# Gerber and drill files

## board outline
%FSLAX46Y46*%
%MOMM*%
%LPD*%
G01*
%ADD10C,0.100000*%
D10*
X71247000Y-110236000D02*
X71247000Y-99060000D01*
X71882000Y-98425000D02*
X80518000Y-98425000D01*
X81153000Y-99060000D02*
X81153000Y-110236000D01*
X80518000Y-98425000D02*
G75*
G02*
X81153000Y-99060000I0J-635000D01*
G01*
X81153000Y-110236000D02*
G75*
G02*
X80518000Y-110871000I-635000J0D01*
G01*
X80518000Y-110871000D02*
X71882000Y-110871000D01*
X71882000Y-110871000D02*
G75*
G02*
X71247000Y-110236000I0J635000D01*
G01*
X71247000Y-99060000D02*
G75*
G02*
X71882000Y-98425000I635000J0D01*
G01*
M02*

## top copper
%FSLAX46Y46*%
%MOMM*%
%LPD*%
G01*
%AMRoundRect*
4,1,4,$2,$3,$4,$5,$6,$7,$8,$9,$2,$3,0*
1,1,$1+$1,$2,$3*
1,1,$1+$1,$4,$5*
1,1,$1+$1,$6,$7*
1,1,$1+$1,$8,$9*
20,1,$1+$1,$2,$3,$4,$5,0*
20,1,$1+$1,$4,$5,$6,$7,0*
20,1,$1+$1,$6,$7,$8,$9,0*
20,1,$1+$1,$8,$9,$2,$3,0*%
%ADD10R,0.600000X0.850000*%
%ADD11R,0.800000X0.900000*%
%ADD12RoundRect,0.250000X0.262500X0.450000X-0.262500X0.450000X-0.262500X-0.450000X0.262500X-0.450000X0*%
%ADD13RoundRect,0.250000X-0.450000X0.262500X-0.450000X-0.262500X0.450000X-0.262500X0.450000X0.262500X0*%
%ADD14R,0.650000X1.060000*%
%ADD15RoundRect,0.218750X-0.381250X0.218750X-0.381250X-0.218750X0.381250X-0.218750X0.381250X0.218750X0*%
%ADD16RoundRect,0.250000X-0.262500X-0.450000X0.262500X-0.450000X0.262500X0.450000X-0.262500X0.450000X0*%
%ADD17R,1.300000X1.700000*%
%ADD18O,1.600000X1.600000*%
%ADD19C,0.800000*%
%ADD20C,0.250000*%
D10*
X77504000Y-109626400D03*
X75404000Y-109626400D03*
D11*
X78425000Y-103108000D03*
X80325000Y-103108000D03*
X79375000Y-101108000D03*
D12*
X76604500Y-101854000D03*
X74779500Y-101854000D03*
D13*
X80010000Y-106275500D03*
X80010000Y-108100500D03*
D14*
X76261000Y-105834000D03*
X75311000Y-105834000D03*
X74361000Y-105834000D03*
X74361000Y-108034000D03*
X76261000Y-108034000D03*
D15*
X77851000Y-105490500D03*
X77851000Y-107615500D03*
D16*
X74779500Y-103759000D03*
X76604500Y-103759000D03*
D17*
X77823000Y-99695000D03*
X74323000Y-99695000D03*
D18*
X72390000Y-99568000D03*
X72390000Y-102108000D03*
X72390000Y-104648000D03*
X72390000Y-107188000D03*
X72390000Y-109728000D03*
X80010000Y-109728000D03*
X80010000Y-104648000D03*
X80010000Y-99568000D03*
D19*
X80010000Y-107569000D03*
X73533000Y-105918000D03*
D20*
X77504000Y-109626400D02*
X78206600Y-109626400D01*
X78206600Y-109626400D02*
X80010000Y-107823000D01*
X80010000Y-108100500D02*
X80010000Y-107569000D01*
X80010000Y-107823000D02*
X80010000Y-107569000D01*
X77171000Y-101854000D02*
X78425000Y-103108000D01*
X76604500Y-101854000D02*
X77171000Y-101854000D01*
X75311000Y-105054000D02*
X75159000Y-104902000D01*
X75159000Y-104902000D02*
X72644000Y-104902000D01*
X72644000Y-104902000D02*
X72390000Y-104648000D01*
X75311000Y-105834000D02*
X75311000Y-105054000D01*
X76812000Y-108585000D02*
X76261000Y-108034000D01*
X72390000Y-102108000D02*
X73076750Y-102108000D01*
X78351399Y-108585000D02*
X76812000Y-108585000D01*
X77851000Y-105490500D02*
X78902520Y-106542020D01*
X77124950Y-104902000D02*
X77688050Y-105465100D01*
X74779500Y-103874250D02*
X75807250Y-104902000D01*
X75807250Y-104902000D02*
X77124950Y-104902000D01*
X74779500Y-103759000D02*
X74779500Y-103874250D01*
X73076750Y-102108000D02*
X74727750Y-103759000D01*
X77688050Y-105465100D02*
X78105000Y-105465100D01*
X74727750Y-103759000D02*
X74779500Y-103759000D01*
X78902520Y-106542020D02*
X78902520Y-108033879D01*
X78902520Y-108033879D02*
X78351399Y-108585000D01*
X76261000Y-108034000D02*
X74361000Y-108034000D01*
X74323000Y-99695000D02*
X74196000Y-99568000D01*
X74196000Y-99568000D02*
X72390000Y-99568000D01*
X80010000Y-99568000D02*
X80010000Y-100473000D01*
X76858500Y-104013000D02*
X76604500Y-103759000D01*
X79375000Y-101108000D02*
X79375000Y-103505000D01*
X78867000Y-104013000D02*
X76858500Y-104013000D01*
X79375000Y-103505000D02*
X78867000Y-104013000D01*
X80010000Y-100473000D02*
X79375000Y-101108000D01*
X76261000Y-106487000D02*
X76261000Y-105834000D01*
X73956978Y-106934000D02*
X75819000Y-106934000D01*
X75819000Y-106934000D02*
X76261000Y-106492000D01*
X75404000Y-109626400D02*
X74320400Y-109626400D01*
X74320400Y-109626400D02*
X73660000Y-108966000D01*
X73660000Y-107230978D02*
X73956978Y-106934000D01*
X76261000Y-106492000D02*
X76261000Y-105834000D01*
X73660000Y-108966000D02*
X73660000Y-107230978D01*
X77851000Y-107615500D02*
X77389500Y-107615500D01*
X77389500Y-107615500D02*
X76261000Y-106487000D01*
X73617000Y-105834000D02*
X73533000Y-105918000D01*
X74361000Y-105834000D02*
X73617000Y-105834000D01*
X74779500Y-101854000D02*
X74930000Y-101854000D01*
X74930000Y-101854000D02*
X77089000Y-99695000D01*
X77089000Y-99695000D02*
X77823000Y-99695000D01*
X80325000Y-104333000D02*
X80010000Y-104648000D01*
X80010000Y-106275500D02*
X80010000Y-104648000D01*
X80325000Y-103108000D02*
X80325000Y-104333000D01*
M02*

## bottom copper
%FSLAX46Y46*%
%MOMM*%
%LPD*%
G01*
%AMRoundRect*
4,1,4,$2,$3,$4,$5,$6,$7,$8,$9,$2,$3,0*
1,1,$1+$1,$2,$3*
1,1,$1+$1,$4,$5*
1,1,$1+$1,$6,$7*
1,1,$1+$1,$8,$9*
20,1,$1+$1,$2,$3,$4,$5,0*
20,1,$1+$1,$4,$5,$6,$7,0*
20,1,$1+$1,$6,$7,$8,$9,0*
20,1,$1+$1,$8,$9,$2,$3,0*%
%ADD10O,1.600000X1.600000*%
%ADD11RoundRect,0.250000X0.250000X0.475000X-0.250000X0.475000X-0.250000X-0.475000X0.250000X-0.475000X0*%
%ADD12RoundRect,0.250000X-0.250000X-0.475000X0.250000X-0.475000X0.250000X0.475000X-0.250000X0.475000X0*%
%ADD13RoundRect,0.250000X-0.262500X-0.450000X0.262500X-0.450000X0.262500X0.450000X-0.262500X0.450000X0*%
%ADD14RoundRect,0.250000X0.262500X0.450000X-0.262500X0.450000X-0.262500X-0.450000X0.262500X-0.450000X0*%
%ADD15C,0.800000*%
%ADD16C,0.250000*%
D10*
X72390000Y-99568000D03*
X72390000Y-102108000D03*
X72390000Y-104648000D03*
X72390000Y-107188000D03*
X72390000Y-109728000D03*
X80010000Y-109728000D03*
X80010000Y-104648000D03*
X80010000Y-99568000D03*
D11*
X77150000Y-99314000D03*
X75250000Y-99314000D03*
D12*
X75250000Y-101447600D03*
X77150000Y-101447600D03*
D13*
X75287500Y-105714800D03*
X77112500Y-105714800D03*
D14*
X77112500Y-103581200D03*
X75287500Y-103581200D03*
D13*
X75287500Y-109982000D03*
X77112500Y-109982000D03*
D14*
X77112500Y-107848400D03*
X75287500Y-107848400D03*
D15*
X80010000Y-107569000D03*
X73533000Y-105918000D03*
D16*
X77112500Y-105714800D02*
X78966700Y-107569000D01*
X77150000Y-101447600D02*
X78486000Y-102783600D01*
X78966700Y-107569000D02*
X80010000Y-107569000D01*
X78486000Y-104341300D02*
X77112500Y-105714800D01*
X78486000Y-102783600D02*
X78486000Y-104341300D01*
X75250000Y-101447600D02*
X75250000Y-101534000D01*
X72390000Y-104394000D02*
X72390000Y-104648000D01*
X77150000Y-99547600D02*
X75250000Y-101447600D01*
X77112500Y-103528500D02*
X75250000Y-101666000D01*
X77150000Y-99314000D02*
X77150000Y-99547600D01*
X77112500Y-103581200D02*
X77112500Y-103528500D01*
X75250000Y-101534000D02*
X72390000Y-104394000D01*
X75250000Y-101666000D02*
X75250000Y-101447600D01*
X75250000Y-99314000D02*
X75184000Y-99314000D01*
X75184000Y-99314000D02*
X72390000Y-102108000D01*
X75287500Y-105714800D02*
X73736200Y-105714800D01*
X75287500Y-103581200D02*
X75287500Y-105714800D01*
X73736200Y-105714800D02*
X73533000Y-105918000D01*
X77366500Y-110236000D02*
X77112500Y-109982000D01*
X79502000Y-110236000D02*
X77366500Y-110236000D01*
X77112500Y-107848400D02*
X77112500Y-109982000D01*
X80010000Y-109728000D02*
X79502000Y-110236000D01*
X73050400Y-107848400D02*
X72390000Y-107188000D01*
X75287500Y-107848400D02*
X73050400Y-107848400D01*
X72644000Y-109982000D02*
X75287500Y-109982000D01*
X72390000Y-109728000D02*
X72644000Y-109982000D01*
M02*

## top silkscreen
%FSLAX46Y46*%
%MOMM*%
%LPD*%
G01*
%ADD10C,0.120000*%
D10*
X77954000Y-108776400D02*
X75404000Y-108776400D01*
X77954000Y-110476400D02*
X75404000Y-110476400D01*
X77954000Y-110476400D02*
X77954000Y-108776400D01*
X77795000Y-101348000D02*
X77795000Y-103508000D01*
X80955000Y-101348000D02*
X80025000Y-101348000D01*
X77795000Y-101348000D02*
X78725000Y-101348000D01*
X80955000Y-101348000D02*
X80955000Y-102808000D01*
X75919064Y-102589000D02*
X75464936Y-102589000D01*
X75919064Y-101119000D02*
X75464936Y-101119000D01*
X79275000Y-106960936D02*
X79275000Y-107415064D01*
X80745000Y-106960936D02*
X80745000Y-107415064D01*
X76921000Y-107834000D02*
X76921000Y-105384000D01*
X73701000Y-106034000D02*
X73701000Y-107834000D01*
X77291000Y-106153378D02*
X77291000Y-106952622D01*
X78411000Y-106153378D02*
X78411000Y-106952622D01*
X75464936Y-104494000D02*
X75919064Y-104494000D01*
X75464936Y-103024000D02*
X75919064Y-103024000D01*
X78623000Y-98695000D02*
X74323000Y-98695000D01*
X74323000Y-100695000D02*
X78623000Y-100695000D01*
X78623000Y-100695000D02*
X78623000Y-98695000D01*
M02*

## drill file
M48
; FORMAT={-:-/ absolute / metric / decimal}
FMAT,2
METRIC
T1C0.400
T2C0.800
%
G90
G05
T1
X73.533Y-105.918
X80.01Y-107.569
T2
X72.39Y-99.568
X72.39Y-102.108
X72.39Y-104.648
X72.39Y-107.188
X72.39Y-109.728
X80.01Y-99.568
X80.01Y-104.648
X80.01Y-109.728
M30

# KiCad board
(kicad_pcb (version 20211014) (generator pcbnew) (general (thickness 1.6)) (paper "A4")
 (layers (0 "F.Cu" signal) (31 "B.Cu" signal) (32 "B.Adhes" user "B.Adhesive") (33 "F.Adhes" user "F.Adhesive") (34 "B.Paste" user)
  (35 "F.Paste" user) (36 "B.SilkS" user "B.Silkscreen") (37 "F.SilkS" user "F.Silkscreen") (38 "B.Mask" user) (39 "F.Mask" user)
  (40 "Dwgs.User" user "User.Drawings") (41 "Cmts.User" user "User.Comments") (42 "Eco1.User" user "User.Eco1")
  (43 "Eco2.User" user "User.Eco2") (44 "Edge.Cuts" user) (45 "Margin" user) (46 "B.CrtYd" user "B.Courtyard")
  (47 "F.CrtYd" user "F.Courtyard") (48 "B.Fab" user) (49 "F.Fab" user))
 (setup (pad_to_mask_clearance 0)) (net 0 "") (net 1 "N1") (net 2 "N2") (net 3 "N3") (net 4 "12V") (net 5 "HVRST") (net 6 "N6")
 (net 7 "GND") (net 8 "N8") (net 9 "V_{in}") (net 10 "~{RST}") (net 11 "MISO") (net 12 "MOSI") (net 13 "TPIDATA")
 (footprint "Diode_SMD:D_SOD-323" (layer "F.Cu") (at 76.454 109.6264 180)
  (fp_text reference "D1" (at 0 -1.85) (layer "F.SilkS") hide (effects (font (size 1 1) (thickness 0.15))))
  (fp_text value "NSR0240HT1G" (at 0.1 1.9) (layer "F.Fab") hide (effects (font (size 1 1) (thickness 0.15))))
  (fp_line (start -1.5 0.85) (end 1.05 0.85) (layer "F.SilkS") (width 0.12))
  (fp_line (start -1.5 -0.85) (end 1.05 -0.85) (layer "F.SilkS") (width 0.12))
  (fp_line (start -1.5 -0.85) (end -1.5 0.85) (layer "F.SilkS") (width 0.12))
  (pad "1" smd rect locked (at -1.05 0 180) (size 0.6 0.85) (layers "F.Cu" "F.Paste" "F.Mask") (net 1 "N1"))
  (pad "2" smd rect locked (at 1.05 0 180) (size 0.6 0.85) (layers "F.Cu" "F.Paste" "F.Mask") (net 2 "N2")))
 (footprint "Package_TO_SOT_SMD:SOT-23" (layer "F.Cu") (at 79.375 102.108 90)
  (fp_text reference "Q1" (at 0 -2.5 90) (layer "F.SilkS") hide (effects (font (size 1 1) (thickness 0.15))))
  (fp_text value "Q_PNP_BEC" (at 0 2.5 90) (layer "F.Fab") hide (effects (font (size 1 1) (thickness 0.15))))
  (fp_line (start 0.76 -1.58) (end -1.4 -1.58) (layer "F.SilkS") (width 0.12))
  (fp_line (start 0.76 1.58) (end 0.76 0.65) (layer "F.SilkS") (width 0.12))
  (fp_line (start 0.76 -1.58) (end 0.76 -0.65) (layer "F.SilkS") (width 0.12))
  (fp_line (start 0.76 1.58) (end -0.7 1.58) (layer "F.SilkS") (width 0.12))
  (pad "1" smd rect locked (at -1 -0.95 90) (size 0.9 0.8) (layers "F.Cu" "F.Paste" "F.Mask") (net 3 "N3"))
  (pad "2" smd rect locked (at -1 0.95 90) (size 0.9 0.8) (layers "F.Cu" "F.Paste" "F.Mask") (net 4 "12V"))
  (pad "3" smd rect locked (at 1 0 90) (size 0.9 0.8) (layers "F.Cu" "F.Paste" "F.Mask") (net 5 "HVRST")))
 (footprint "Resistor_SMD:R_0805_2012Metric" (layer "F.Cu") (at 75.692 101.854 180)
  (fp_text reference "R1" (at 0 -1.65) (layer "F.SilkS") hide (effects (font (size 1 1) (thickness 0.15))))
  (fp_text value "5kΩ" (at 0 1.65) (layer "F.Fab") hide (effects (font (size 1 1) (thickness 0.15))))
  (fp_line (start -0.227064 -0.735) (end 0.227064 -0.735) (layer "F.SilkS") (width 0.12))
  (fp_line (start -0.227064 0.735) (end 0.227064 0.735) (layer "F.SilkS") (width 0.12))
  (pad "1" smd roundrect locked (at -0.9125 0 180) (size 1.025 1.4) (layers "F.Cu" "F.Paste" "F.Mask") (roundrect_rratio 0.243902)
   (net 3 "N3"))
  (pad "2" smd roundrect locked (at 0.9125 0 180) (size 1.025 1.4) (layers "F.Cu" "F.Paste" "F.Mask") (roundrect_rratio 0.243902)
   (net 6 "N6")))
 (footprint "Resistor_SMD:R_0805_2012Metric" (layer "F.Cu") (at 80.01 107.188 -90)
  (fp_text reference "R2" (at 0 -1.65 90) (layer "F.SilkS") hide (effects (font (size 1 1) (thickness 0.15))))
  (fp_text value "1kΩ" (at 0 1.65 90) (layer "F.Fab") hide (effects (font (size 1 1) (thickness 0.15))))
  (fp_line (start -0.227064 0.735) (end 0.227064 0.735) (layer "F.SilkS") (width 0.12))
  (fp_line (start -0.227064 -0.735) (end 0.227064 -0.735) (layer "F.SilkS") (width 0.12))
  (pad "1" smd roundrect locked (at -0.9125 0 270) (size 1.025 1.4) (layers "F.Cu" "F.Paste" "F.Mask") (roundrect_rratio 0.243902)
   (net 4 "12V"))
  (pad "2" smd roundrect locked (at 0.9125 0 270) (size 1.025 1.4) (layers "F.Cu" "F.Paste" "F.Mask") (roundrect_rratio 0.243902)
   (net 1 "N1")))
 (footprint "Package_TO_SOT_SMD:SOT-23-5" (layer "F.Cu") (at 75.311 106.934 -90)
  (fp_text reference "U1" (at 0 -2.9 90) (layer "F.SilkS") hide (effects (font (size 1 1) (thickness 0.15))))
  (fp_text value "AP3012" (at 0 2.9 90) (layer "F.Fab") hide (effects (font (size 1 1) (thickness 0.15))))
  (fp_line (start 0.9 -1.61) (end -1.55 -1.61) (layer "F.SilkS") (width 0.12))
  (fp_line (start -0.9 1.61) (end 0.9 1.61) (layer "F.SilkS") (width 0.12))
  (pad "1" smd rect locked (at -1.1 -0.95 270) (size 1.06 0.65) (layers "F.Cu" "F.Paste" "F.Mask") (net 2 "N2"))
  (pad "2" smd rect locked (at -1.1 0 270) (size 1.06 0.65) (layers "F.Cu" "F.Paste" "F.Mask") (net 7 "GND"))
  (pad "3" smd rect locked (at -1.1 0.95 270) (size 1.06 0.65) (layers "F.Cu" "F.Paste" "F.Mask") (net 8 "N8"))
  (pad "4" smd rect locked (at 1.1 0.95 270) (size 1.06 0.65) (layers "F.Cu" "F.Paste" "F.Mask") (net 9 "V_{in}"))
  (pad "5" smd rect locked (at 1.1 -0.95 270) (size 1.06 0.65) (layers "F.Cu" "F.Paste" "F.Mask") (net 9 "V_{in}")))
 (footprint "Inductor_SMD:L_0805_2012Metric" (layer "F.Cu") (at 77.851 106.553 -90)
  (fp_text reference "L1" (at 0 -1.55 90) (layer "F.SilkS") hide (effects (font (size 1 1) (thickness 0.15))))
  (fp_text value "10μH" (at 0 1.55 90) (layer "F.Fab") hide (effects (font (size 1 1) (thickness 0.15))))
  (fp_line (start -0.399622 0.56) (end 0.399622 0.56) (layer "F.SilkS") (width 0.12))
  (fp_line (start -0.399622 -0.56) (end 0.399622 -0.56) (layer "F.SilkS") (width 0.12))
  (pad "1" smd roundrect locked (at -1.0625 0 270) (size 0.875 1.2) (layers "F.Cu" "F.Paste" "F.Mask") (roundrect_rratio 0.25)
   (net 9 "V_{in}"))
  (pad "2" smd roundrect locked (at 1.0625 0 270) (size 0.875 1.2) (layers "F.Cu" "F.Paste" "F.Mask") (roundrect_rratio 0.25) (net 2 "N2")))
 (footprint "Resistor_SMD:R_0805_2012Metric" (layer "F.Cu") (at 75.692 103.759)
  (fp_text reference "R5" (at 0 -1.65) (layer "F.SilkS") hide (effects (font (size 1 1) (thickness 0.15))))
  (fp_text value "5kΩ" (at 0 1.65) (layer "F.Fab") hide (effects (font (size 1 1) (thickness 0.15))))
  (fp_line (start -0.227064 0.735) (end 0.227064 0.735) (layer "F.SilkS") (width 0.12))
  (fp_line (start -0.227064 -0.735) (end 0.227064 -0.735) (layer "F.SilkS") (width 0.12))
  (pad "1" smd roundrect locked (at -0.9125 0) (size 1.025 1.4) (layers "F.Cu" "F.Paste" "F.Mask") (roundrect_rratio 0.243902)
   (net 9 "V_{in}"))
  (pad "2" smd roundrect locked (at 0.9125 0) (size 1.025 1.4) (layers "F.Cu" "F.Paste" "F.Mask") (roundrect_rratio 0.243902)
   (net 5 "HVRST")))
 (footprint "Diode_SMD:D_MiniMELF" (layer "F.Cu") (at 76.073 99.695 180)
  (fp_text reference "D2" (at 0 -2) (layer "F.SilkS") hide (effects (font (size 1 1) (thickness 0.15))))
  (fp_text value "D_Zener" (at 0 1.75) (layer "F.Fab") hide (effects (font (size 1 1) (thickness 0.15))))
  (fp_line (start -2.55 1) (end 1.75 1) (layer "F.SilkS") (width 0.12))
  (fp_line (start 1.75 -1) (end -2.55 -1) (layer "F.SilkS") (width 0.12))
  (fp_line (start -2.55 -1) (end -2.55 1) (layer "F.SilkS") (width 0.12))
  (pad "1" smd rect locked (at -1.75 0 180) (size 1.3 1.7) (layers "F.Cu" "F.Paste" "F.Mask") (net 6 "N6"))
  (pad "2" smd rect locked (at 1.75 0 180) (size 1.3 1.7) (layers "F.Cu" "F.Paste" "F.Mask") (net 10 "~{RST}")))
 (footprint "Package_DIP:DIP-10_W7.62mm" (layer "F.Cu") (at 72.39 99.568)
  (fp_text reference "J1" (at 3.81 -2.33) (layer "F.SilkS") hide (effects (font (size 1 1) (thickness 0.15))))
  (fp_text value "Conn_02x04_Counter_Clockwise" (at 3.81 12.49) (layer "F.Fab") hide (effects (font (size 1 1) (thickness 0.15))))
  (pad "1" thru_hole oval (at 0 0) (size 1.6 1.6) (drill 0.8) (layers *.Cu *.Mask) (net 10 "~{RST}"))
  (pad "2" thru_hole oval (at 0 2.54) (size 1.6 1.6) (drill 0.8) (layers *.Cu *.Mask) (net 9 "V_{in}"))
  (pad "3" thru_hole oval (at 0 5.08) (size 1.6 1.6) (drill 0.8) (layers *.Cu *.Mask) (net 7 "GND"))
  (pad "4" thru_hole oval (at 0 7.62) (size 1.6 1.6) (drill 0.8) (layers *.Cu *.Mask) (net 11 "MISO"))
  (pad "5" thru_hole oval (at 0 10.16) (size 1.6 1.6) (drill 0.8) (layers *.Cu *.Mask) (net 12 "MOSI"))
  (pad "6" thru_hole oval (at 7.62 10.16) (size 1.6 1.6) (drill 0.8) (layers *.Cu *.Mask) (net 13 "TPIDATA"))
  (pad "8" thru_hole oval (at 7.62 5.08) (size 1.6 1.6) (drill 0.8) (layers *.Cu *.Mask) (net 4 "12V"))
  (pad "10" thru_hole oval (at 7.62 0) (size 1.6 1.6) (drill 0.8) (layers *.Cu *.Mask) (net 5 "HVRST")))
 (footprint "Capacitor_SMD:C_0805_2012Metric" (layer "B.Cu") (at 76.2 99.314 180)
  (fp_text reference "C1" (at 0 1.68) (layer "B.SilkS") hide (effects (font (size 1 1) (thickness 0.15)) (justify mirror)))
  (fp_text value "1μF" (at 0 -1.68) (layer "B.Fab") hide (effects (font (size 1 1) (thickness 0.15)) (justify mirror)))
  (pad "1" smd roundrect locked (at -0.95 0 180) (size 1 1.45) (layers "B.Cu" "B.Paste" "B.Mask") (roundrect_rratio 0.25) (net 7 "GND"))
  (pad "2" smd roundrect locked (at 0.95 0 180) (size 1 1.45) (layers "B.Cu" "B.Paste" "B.Mask") (roundrect_rratio 0.25) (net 9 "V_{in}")))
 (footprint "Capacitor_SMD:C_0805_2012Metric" (layer "B.Cu") (at 76.2 101.4476)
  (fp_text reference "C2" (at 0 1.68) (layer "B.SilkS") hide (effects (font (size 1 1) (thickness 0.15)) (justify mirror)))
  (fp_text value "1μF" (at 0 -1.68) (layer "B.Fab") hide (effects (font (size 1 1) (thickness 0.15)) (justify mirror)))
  (pad "1" smd roundrect locked (at -0.95 0) (size 1 1.45) (layers "B.Cu" "B.Paste" "B.Mask") (roundrect_rratio 0.25) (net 7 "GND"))
  (pad "2" smd roundrect locked (at 0.95 0) (size 1 1.45) (layers "B.Cu" "B.Paste" "B.Mask") (roundrect_rratio 0.25) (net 1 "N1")))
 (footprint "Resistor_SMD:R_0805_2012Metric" (layer "B.Cu") (at 76.2 105.7148)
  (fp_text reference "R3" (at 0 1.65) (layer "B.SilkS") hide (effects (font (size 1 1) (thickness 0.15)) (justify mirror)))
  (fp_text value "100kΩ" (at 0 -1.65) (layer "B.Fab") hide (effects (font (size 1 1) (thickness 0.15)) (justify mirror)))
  (pad "1" smd roundrect locked (at -0.9125 0) (size 1.025 1.4) (layers "B.Cu" "B.Paste" "B.Mask") (roundrect_rratio 0.243902) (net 8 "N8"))
  (pad "2" smd roundrect locked (at 0.9125 0) (size 1.025 1.4) (layers "B.Cu" "B.Paste" "B.Mask") (roundrect_rratio 0.243902) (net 1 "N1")))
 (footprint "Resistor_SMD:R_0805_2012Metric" (layer "B.Cu") (at 76.2 103.5812 180)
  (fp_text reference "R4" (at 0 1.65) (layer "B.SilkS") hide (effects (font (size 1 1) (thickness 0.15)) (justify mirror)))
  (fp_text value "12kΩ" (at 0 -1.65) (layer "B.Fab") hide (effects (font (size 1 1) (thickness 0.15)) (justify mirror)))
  (pad "1" smd roundrect locked (at -0.9125 0 180) (size 1.025 1.4) (layers "B.Cu" "B.Paste" "B.Mask") (roundrect_rratio 0.243902)
   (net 7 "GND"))
  (pad "2" smd roundrect locked (at 0.9125 0 180) (size 1.025 1.4) (layers "B.Cu" "B.Paste" "B.Mask") (roundrect_rratio 0.243902)
   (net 8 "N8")))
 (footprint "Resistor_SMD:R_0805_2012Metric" (layer "B.Cu") (at 76.2 109.982)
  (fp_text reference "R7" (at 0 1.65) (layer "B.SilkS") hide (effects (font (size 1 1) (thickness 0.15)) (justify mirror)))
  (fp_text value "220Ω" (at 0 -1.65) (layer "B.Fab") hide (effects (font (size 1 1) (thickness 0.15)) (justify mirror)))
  (pad "1" smd roundrect (at -0.9125 0) (size 1.025 1.4) (layers "B.Cu" "B.Paste" "B.Mask") (roundrect_rratio 0.243902) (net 12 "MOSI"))
  (pad "2" smd roundrect (at 0.9125 0) (size 1.025 1.4) (layers "B.Cu" "B.Paste" "B.Mask") (roundrect_rratio 0.243902) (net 13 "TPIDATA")))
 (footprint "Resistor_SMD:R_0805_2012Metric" (layer "B.Cu") (at 76.2 107.8484 180)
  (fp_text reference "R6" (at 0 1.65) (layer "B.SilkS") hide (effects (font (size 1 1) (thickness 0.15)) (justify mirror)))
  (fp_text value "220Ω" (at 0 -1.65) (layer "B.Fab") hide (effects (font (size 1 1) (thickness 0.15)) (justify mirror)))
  (pad "1" smd roundrect (at -0.9125 0 180) (size 1.025 1.4) (layers "B.Cu" "B.Paste" "B.Mask") (roundrect_rratio 0.243902)
   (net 13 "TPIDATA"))
  (pad "2" smd roundrect (at 0.9125 0 180) (size 1.025 1.4) (layers "B.Cu" "B.Paste" "B.Mask") (roundrect_rratio 0.243902) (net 11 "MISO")))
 (gr_line (start 71.247 110.236) (end 71.247 99.06) (layer "Edge.Cuts") (width 0.1))
 (gr_line (start 71.882 98.425) (end 80.518 98.425) (layer "Edge.Cuts") (width 0.1))
 (gr_line (start 81.153 99.06) (end 81.153 110.236) (layer "Edge.Cuts") (width 0.1))
 (gr_arc (start 80.518 98.425) (mid 80.967013 98.610987) (end 81.153 99.06) (layer "Edge.Cuts") (width 0.1))
 (gr_arc (start 81.153 110.236) (mid 80.967013 110.685013) (end 80.518 110.871) (layer "Edge.Cuts") (width 0.1))
 (gr_line (start 80.518 110.871) (end 71.882 110.871) (layer "Edge.Cuts") (width 0.1))
 (gr_arc (start 71.882 110.871) (mid 71.432987 110.685013) (end 71.247 110.236) (layer "Edge.Cuts") (width 0.1))
 (gr_arc (start 71.247 99.06) (mid 71.432987 98.610987) (end 71.882 98.425) (layer "Edge.Cuts") (width 0.1))
 (segment (start 77.504 109.6264) (end 78.2066 109.6264) (width 0.25) (layer "F.Cu") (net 1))
 (segment (start 78.2066 109.6264) (end 80.01 107.823) (width 0.25) (layer "F.Cu") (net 1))
 (segment (start 80.01 108.1005) (end 80.01 107.569) (width 0.25) (layer "F.Cu") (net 1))
 (segment (start 80.01 107.823) (end 80.01 107.569) (width 0.25) (layer "F.Cu") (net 1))
 (via (at 80.01 107.569) (size 0.8) (drill 0.4) (layers "F.Cu" "B.Cu") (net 1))
 (segment (start 77.1125 105.7148) (end 78.9667 107.569) (width 0.25) (layer "B.Cu") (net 1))
 (segment (start 77.15 101.4476) (end 78.486 102.7836) (width 0.25) (layer "B.Cu") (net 1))
 (segment (start 78.9667 107.569) (end 80.01 107.569) (width 0.25) (layer "B.Cu") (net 1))
 (segment (start 78.486 104.3413) (end 77.1125 105.7148) (width 0.25) (layer "B.Cu") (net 1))
 (segment (start 78.486 102.7836) (end 78.486 104.3413) (width 0.25) (layer "B.Cu") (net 1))
 (segment (start 77.171 101.854) (end 78.425 103.108) (width 0.25) (layer "F.Cu") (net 3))
 (segment (start 76.6045 101.854) (end 77.171 101.854) (width 0.25) (layer "F.Cu") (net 3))
 (segment (start 75.311 105.054) (end 75.159 104.902) (width 0.25) (layer "F.Cu") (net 7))
 (segment (start 75.159 104.902) (end 72.644 104.902) (width 0.25) (layer "F.Cu") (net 7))
 (segment (start 72.644 104.902) (end 72.39 104.648) (width 0.25) (layer "F.Cu") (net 7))
 (segment (start 75.311 105.834) (end 75.311 105.054) (width 0.25) (layer "F.Cu") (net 7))
 (segment (start 75.25 101.4476) (end 75.25 101.534) (width 0.25) (layer "B.Cu") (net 7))
 (segment (start 72.39 104.394) (end 72.39 104.648) (width 0.25) (layer "B.Cu") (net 7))
 (segment (start 77.15 99.5476) (end 75.25 101.4476) (width 0.25) (layer "B.Cu") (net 7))
 (segment (start 77.1125 103.5285) (end 75.25 101.666) (width 0.25) (layer "B.Cu") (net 7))
 (segment (start 77.15 99.314) (end 77.15 99.5476) (width 0.25) (layer "B.Cu") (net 7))
 (segment (start 77.1125 103.5812) (end 77.1125 103.5285) (width 0.25) (layer "B.Cu") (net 7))
 (segment (start 75.25 101.534) (end 72.39 104.394) (width 0.25) (layer "B.Cu") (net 7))
 (segment (start 75.25 101.666) (end 75.25 101.4476) (width 0.25) (layer "B.Cu") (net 7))
 (segment (start 76.812 108.585) (end 76.261 108.034) (width 0.25) (layer "F.Cu") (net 9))
 (segment (start 72.39 102.108) (end 73.07675 102.108) (width 0.25) (layer "F.Cu") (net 9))
 (segment (start 78.351399 108.585) (end 76.812 108.585) (width 0.25) (layer "F.Cu") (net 9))
 (segment (start 77.851 105.4905) (end 78.90252 106.54202) (width 0.25) (layer "F.Cu") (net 9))
 (segment (start 77.12495 104.902) (end 77.68805 105.4651) (width 0.25) (layer "F.Cu") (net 9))
 (segment (start 74.7795 103.87425) (end 75.80725 104.902) (width 0.25) (layer "F.Cu") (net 9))
 (segment (start 75.80725 104.902) (end 77.12495 104.902) (width 0.25) (layer "F.Cu") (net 9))
 (segment (start 74.7795 103.759) (end 74.7795 103.87425) (width 0.25) (layer "F.Cu") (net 9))
 (segment (start 73.07675 102.108) (end 74.72775 103.759) (width 0.25) (layer "F.Cu") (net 9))
 (segment (start 77.68805 105.4651) (end 78.105 105.4651) (width 0.25) (layer "F.Cu") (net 9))
 (segment (start 74.72775 103.759) (end 74.7795 103.759) (width 0.25) (layer "F.Cu") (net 9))
 (segment (start 78.90252 106.54202) (end 78.90252 108.033879) (width 0.25) (layer "F.Cu") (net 9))
 (segment (start 78.90252 108.033879) (end 78.351399 108.585) (width 0.25) (layer "F.Cu") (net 9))
 (segment (start 76.261 108.034) (end 74.361 108.034) (width 0.25) (layer "F.Cu") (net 9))
 (segment (start 75.25 99.314) (end 75.184 99.314) (width 0.25) (layer "B.Cu") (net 9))
 (segment (start 75.184 99.314) (end 72.39 102.108) (width 0.25) (layer "B.Cu") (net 9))
 (segment (start 74.323 99.695) (end 74.196 99.568) (width 0.25) (layer "F.Cu") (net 10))
 (segment (start 74.196 99.568) (end 72.39 99.568) (width 0.25) (layer "F.Cu") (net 10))
 (segment (start 80.01 99.568) (end 80.01 100.473) (width 0.25) (layer "F.Cu") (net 5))
 (segment (start 76.8585 104.013) (end 76.6045 103.759) (width 0.25) (layer "F.Cu") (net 5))
 (segment (start 79.375 101.108) (end 79.375 103.505) (width 0.25) (layer "F.Cu") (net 5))
 (segment (start 78.867 104.013) (end 76.8585 104.013) (width 0.25) (layer "F.Cu") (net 5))
 (segment (start 79.375 103.505) (end 78.867 104.013) (width 0.25) (layer "F.Cu") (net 5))
 (segment (start 80.01 100.473) (end 79.375 101.108) (width 0.25) (layer "F.Cu") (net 5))
 (segment (start 76.261 106.487) (end 76.261 105.834) (width 0.25) (layer "F.Cu") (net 2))
 (segment (start 73.956978 106.934) (end 75.819 106.934) (width 0.25) (layer "F.Cu") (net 2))
 (segment (start 75.819 106.934) (end 76.261 106.492) (width 0.25) (layer "F.Cu") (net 2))
 (segment (start 75.404 109.6264) (end 74.3204 109.6264) (width 0.25) (layer "F.Cu") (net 2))
 (segment (start 74.3204 109.6264) (end 73.66 108.966) (width 0.25) (layer "F.Cu") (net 2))
 (segment (start 73.66 107.230978) (end 73.956978 106.934) (width 0.25) (layer "F.Cu") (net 2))
 (segment (start 76.261 106.492) (end 76.261 105.834) (width 0.25) (layer "F.Cu") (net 2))
 (segment (start 73.66 108.966) (end 73.66 107.230978) (width 0.25) (layer "F.Cu") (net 2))
 (segment (start 77.851 107.6155) (end 77.3895 107.6155) (width 0.25) (layer "F.Cu") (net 2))
 (segment (start 77.3895 107.6155) (end 76.261 106.487) (width 0.25) (layer "F.Cu") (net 2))
 (segment (start 73.617 105.834) (end 73.533 105.918) (width 0.25) (layer "F.Cu") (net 8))
 (segment (start 74.361 105.834) (end 73.617 105.834) (width 0.25) (layer "F.Cu") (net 8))
 (via (at 73.533 105.918) (size 0.8) (drill 0.4) (layers "F.Cu" "B.Cu") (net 8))
 (segment (start 75.2875 105.7148) (end 73.7362 105.7148) (width 0.25) (layer "B.Cu") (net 8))
 (segment (start 75.2875 103.5812) (end 75.2875 105.7148) (width 0.25) (layer "B.Cu") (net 8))
 (segment (start 73.7362 105.7148) (end 73.533 105.918) (width 0.25) (layer "B.Cu") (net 8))
 (segment (start 74.7795 101.854) (end 74.93 101.854) (width 0.25) (layer "F.Cu") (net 6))
 (segment (start 74.93 101.854) (end 77.089 99.695) (width 0.25) (layer "F.Cu") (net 6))
 (segment (start 77.089 99.695) (end 77.823 99.695) (width 0.25) (layer "F.Cu") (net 6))
 (segment (start 80.325 104.333) (end 80.01 104.648) (width 0.25) (layer "F.Cu") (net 4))
 (segment (start 80.01 106.2755) (end 80.01 104.648) (width 0.25) (layer "F.Cu") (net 4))
 (segment (start 80.325 103.108) (end 80.325 104.333) (width 0.25) (layer "F.Cu") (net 4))
 (segment (start 77.3665 110.236) (end 77.1125 109.982) (width 0.25) (layer "B.Cu") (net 13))
 (segment (start 79.502 110.236) (end 77.3665 110.236) (width 0.25) (layer "B.Cu") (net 13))
 (segment (start 77.1125 107.8484) (end 77.1125 109.982) (width 0.25) (layer "B.Cu") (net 13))
 (segment (start 80.01 109.728) (end 79.502 110.236) (width 0.25) (layer "B.Cu") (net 13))
 (segment (start 73.0504 107.8484) (end 72.39 107.188) (width 0.25) (layer "B.Cu") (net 11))
 (segment (start 75.2875 107.8484) (end 73.0504 107.8484) (width 0.25) (layer "B.Cu") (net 11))
 (segment (start 72.644 109.982) (end 75.2875 109.982) (width 0.25) (layer "B.Cu") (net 12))
 (segment (start 72.39 109.728) (end 72.644 109.982) (width 0.25) (layer "B.Cu") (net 12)))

